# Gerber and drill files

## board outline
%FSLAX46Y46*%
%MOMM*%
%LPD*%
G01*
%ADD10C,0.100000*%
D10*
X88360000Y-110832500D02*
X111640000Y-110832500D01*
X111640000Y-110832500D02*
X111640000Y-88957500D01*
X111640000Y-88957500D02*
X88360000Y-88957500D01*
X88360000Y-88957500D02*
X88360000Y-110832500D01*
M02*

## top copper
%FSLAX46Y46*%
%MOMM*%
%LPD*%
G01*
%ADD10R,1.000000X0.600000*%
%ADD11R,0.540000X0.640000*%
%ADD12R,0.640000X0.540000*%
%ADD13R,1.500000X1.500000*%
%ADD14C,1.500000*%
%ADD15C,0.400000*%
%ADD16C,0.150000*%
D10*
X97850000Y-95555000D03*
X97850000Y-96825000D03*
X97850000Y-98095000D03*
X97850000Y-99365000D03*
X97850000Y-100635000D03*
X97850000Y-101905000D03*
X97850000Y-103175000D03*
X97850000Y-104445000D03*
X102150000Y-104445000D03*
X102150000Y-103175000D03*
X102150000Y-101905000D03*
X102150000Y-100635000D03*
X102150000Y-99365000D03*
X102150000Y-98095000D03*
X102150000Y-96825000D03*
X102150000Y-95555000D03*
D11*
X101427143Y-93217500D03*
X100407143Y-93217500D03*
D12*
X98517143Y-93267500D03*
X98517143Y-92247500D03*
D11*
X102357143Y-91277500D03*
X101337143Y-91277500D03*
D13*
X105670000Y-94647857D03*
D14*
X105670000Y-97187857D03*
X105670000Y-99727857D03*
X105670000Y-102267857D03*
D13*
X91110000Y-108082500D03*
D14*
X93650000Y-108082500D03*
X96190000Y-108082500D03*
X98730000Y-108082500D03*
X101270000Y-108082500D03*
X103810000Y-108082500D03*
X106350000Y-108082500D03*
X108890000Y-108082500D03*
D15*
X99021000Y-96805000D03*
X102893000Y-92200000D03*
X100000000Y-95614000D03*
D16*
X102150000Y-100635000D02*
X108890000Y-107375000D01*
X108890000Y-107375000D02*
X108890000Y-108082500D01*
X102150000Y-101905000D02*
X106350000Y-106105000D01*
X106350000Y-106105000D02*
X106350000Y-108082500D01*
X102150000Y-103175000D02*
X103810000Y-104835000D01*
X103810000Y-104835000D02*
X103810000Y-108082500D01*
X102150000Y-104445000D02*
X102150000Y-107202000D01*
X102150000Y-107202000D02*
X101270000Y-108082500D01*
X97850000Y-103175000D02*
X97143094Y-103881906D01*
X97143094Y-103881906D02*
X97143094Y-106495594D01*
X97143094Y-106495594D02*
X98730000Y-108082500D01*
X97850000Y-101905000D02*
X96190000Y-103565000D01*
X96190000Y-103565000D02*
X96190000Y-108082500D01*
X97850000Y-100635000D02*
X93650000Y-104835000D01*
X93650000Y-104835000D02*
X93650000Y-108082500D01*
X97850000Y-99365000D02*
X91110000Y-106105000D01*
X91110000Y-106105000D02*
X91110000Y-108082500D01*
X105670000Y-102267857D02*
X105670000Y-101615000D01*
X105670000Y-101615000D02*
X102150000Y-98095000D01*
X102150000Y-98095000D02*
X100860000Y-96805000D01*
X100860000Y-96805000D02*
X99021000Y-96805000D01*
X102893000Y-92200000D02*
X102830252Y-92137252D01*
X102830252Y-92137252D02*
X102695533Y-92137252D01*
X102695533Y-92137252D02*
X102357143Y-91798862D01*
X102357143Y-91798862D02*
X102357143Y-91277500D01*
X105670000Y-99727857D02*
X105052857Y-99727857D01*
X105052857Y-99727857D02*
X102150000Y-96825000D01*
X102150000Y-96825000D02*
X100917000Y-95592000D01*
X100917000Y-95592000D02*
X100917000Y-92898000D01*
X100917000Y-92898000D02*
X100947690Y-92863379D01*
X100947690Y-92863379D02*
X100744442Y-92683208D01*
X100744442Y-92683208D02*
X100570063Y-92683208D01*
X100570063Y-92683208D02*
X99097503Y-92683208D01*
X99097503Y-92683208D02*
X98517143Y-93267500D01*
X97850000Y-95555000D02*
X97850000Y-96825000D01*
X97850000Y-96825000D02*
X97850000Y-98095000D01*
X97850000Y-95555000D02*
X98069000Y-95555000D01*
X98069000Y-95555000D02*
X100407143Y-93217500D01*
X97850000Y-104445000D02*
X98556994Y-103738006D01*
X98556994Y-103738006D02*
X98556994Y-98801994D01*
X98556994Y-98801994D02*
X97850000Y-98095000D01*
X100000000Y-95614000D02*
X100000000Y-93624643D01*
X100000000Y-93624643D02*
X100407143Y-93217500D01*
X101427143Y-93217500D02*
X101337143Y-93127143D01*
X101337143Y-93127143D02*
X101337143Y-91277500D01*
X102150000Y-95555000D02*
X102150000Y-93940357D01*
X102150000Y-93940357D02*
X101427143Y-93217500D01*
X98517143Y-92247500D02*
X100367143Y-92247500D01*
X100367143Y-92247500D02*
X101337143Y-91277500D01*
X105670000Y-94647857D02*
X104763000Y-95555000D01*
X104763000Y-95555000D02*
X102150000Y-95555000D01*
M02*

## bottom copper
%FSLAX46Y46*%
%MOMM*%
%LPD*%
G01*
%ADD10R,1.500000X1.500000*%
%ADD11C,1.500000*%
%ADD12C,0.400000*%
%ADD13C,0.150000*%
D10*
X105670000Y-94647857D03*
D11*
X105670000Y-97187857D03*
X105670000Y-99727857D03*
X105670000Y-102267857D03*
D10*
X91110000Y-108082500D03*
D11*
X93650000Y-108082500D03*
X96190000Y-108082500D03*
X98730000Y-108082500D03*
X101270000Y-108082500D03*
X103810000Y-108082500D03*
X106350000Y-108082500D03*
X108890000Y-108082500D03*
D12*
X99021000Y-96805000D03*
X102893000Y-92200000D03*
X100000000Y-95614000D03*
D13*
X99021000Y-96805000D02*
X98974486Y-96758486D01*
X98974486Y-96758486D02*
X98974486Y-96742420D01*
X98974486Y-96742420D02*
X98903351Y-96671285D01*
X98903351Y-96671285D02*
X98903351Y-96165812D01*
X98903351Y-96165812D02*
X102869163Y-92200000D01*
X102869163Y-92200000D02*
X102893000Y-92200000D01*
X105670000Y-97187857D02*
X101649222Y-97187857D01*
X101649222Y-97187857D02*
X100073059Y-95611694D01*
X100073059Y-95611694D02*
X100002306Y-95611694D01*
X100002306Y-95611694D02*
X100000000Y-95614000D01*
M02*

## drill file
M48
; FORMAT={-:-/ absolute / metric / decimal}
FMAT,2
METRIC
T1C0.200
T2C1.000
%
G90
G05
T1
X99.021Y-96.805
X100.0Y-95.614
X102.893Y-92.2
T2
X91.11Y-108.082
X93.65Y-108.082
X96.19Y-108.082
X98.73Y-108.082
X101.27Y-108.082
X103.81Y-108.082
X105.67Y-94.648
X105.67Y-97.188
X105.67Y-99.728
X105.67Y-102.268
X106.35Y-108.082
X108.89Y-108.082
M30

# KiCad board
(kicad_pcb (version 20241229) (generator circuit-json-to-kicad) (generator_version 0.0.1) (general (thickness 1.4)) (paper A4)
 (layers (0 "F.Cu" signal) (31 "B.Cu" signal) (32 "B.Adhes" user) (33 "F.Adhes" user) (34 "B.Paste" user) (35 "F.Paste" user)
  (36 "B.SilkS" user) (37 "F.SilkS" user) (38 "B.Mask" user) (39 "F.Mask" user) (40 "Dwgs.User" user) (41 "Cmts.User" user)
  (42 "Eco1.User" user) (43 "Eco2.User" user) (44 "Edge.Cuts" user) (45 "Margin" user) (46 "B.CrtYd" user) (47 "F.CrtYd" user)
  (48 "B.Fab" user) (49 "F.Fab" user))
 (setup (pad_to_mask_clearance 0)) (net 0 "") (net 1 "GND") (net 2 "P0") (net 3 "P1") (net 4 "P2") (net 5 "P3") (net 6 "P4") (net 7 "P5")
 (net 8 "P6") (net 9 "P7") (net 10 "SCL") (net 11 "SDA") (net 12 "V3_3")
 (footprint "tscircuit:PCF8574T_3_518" (layer F.Cu) (at 100 100 0)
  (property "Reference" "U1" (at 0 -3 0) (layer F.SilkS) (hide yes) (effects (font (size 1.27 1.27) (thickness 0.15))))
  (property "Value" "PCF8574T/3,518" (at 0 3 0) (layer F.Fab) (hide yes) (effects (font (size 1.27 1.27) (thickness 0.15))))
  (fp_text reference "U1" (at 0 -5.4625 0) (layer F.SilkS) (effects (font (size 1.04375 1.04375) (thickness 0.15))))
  (pad "1" smd rect (at -2.15 -4.445 0) (size 1 0.6) (layers F.Cu F.Paste F.Mask) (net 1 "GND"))
  (pad "2" smd rect (at -2.15 -3.1750000000000003 0) (size 1 0.6) (layers F.Cu F.Paste F.Mask) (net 1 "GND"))
  (pad "3" smd rect (at -2.15 -1.9050000000000002 0) (size 1 0.6) (layers F.Cu F.Paste F.Mask) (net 1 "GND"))
  (pad "4" smd rect (at -2.15 -0.6350000000000002 0) (size 1 0.6) (layers F.Cu F.Paste F.Mask) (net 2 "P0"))
  (pad "5" smd rect (at -2.15 0.6349999999999998 0) (size 1 0.6) (layers F.Cu F.Paste F.Mask) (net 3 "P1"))
  (pad "6" smd rect (at -2.15 1.9049999999999994 0) (size 1 0.6) (layers F.Cu F.Paste F.Mask) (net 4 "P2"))
  (pad "7" smd rect (at -2.15 3.175 0) (size 1 0.6) (layers F.Cu F.Paste F.Mask) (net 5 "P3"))
  (pad "8" smd rect (at -2.15 4.445 0) (size 1 0.6) (layers F.Cu F.Paste F.Mask) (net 1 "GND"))
  (pad "9" smd rect (at 2.15 4.445 0) (size 1 0.6) (layers F.Cu F.Paste F.Mask) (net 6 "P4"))
  (pad "10" smd rect (at 2.15 3.1750000000000003 0) (size 1 0.6) (layers F.Cu F.Paste F.Mask) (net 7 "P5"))
  (pad "11" smd rect (at 2.15 1.9050000000000002 0) (size 1 0.6) (layers F.Cu F.Paste F.Mask) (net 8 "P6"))
  (pad "12" smd rect (at 2.15 0.6350000000000002 0) (size 1 0.6) (layers F.Cu F.Paste F.Mask) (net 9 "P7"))
  (pad "13" smd rect (at 2.15 -0.6349999999999998 0) (size 1 0.6) (layers F.Cu F.Paste F.Mask))
  (pad "14" smd rect (at 2.15 -1.9049999999999994 0) (size 1 0.6) (layers F.Cu F.Paste F.Mask) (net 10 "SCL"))
  (pad "15" smd rect (at 2.15 -3.175 0) (size 1 0.6) (layers F.Cu F.Paste F.Mask) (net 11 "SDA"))
  (pad "16" smd rect (at 2.15 -4.445 0) (size 1 0.6) (layers F.Cu F.Paste F.Mask) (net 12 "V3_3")))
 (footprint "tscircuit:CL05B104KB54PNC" (layer F.Cu) (at 100.91714285714286 93.2175 180)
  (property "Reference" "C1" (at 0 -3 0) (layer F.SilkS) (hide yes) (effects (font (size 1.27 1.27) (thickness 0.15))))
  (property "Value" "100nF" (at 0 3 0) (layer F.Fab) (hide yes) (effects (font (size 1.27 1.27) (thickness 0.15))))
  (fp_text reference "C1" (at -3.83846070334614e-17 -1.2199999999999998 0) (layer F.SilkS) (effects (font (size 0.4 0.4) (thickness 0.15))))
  (pad "1" smd rect (at -0.5099999999999999 0 0) (size 0.54 0.64) (layers F.Cu F.Paste F.Mask) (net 12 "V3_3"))
  (pad "2" smd rect (at 0.51 0 0) (size 0.54 0.64) (layers F.Cu F.Paste F.Mask) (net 1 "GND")))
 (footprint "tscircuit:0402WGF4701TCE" (layer F.Cu) (at 98.51714285714286 92.7575 90)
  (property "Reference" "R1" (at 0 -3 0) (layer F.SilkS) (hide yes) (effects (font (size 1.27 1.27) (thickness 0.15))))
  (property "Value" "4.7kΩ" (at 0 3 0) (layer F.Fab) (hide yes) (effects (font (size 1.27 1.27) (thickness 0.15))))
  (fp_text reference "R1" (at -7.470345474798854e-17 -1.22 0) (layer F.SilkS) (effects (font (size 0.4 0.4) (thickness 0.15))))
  (pad "1" smd rect (at -0.5099999999999998 0 0) (size 0.64 0.54) (layers F.Cu F.Paste F.Mask) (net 11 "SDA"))
  (pad "2" smd rect (at 0.5099999999999998 0 0) (size 0.64 0.54) (layers F.Cu F.Paste F.Mask) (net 12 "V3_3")))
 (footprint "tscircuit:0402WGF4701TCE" (layer F.Cu) (at 101.84714285714286 91.2775 180)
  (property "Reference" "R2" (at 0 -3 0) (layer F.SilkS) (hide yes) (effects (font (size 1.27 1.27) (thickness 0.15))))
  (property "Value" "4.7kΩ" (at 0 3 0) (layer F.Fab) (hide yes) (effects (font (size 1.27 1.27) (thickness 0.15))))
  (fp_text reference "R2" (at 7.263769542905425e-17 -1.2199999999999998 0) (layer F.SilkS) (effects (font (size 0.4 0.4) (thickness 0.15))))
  (pad "1" smd rect (at -0.51 0 0) (size 0.54 0.64) (layers F.Cu F.Paste F.Mask) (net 10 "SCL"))
  (pad "2" smd rect (at 0.51 0 0) (size 0.54 0.64) (layers F.Cu F.Paste F.Mask) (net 12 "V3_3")))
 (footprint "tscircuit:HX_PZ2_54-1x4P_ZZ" (layer F.Cu) (at 105.67 98.45785714285714 -90.00000000000001)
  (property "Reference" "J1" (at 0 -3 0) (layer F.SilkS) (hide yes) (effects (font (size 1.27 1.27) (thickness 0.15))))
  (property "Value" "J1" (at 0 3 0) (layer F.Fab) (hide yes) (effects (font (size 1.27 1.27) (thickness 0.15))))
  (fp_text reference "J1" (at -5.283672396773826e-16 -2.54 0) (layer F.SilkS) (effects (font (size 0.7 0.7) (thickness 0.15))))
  (pad "1" thru_hole rect (at -3.81 5.705062545910424e-16 0) (size 1.5 1.5) (drill 1) (layers *.Cu *.Mask) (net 12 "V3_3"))
  (pad "2" thru_hole circle (at -1.27 4.862282247637226e-16 0) (size 1.5 1.5) (drill 1) (layers *.Cu *.Mask) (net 1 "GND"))
  (pad "3" thru_hole circle (at 1.27 -4.862282247637226e-16 0) (size 1.5 1.5) (drill 1) (layers *.Cu *.Mask) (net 11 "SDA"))
  (pad "4" thru_hole circle (at 3.81 -5.705062545910424e-16 0) (size 1.5 1.5) (drill 1) (layers *.Cu *.Mask) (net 10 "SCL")))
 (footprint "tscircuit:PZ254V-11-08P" (layer F.Cu) (at 100 108.0825 0)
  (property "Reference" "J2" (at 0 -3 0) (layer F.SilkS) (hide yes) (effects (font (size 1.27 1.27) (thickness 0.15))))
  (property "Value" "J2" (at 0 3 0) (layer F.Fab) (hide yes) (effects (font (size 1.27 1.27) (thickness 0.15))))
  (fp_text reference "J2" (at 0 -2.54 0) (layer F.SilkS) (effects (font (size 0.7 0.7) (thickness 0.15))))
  (pad "1" thru_hole rect (at -8.89 0 0) (size 1.5 1.5) (drill 1) (layers *.Cu *.Mask) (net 2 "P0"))
  (pad "2" thru_hole circle (at -6.3500000000000005 0 0) (size 1.5 1.5) (drill 1) (layers *.Cu *.Mask) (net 3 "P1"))
  (pad "3" thru_hole circle (at -3.8100000000000005 0 0) (size 1.5 1.5) (drill 1) (layers *.Cu *.Mask) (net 4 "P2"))
  (pad "4" thru_hole circle (at -1.2700000000000005 0 0) (size 1.5 1.5) (drill 1) (layers *.Cu *.Mask) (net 5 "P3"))
  (pad "5" thru_hole circle (at 1.2699999999999996 0 0) (size 1.5 1.5) (drill 1) (layers *.Cu *.Mask) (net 6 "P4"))
  (pad "6" thru_hole circle (at 3.8099999999999987 0 0) (size 1.5 1.5) (drill 1) (layers *.Cu *.Mask) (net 7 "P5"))
  (pad "7" thru_hole circle (at 6.35 0 0) (size 1.5 1.5) (drill 1) (layers *.Cu *.Mask) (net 8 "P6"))
  (pad "8" thru_hole circle (at 8.89 0 0) (size 1.5 1.5) (drill 1) (layers *.Cu *.Mask) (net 9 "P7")))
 (segment (start 102.15 100.635) (end 108.89 107.375) (width 0.15) (layer F.Cu) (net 9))
 (segment (start 108.89 107.375) (end 108.89 108.0825) (width 0.15) (layer F.Cu) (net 9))
 (segment (start 102.15 101.905) (end 106.35 106.105) (width 0.15) (layer F.Cu) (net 8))
 (segment (start 106.35 106.105) (end 106.35 108.0825) (width 0.15) (layer F.Cu) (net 8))
 (segment (start 102.15 103.175) (end 103.81 104.835) (width 0.15) (layer F.Cu) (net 7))
 (segment (start 103.81 104.835) (end 103.81 108.0825) (width 0.15) (layer F.Cu) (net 7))
 (segment (start 102.15 104.445) (end 102.15 107.202) (width 0.15) (layer F.Cu) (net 6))
 (segment (start 102.15 107.202) (end 101.27 108.0825) (width 0.15) (layer F.Cu) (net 6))
 (segment (start 97.85 103.175) (end 97.14309387785406 103.88190612214595) (width 0.15) (layer F.Cu) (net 5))
 (segment (start 97.14309387785406 103.88190612214595) (end 97.14309387785406 106.49559387785405) (width 0.15) (layer F.Cu) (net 5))
 (segment (start 97.14309387785406 106.49559387785405) (end 98.73 108.0825) (width 0.15) (layer F.Cu) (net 5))
 (segment (start 97.85 101.905) (end 96.19 103.565) (width 0.15) (layer F.Cu) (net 4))
 (segment (start 96.19 103.565) (end 96.19 108.0825) (width 0.15) (layer F.Cu) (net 4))
 (segment (start 97.85 100.635) (end 93.65 104.83500000000001) (width 0.15) (layer F.Cu) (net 3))
 (segment (start 93.65 104.83500000000001) (end 93.65 108.0825) (width 0.15) (layer F.Cu) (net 3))
 (segment (start 97.85 99.365) (end 91.11 106.105) (width 0.15) (layer F.Cu) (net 2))
 (segment (start 91.11 106.105) (end 91.11 108.0825) (width 0.15) (layer F.Cu) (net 2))
 (segment (start 105.67 102.26785714285714) (end 105.67 101.615) (width 0.15) (layer F.Cu) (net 10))
 (segment (start 105.67 101.615) (end 102.15 98.095) (width 0.15) (layer F.Cu) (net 10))
 (segment (start 102.15 98.095) (end 100.86 96.805) (width 0.15) (layer F.Cu) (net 10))
 (segment (start 100.86 96.805) (end 99.021 96.805) (width 0.15) (layer F.Cu) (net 10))
 (segment (start 99.021 96.805) (end 98.97448570689265 96.75848570689264) (width 0.15) (layer B.Cu) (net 10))
 (segment (start 98.97448570689265 96.75848570689264) (end 98.97448570689265 96.7424195752621) (width 0.15) (layer B.Cu) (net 10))
 (segment (start 98.97448570689265 96.7424195752621) (end 98.90335073935582 96.67128460772527) (width 0.15) (layer B.Cu) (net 10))
 (segment (start 98.90335073935582 96.67128460772527) (end 98.90335073935582 96.1658122704005) (width 0.15) (layer B.Cu) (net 10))
 (segment (start 98.90335073935582 96.1658122704005) (end 102.86916300975629 92.2) (width 0.15) (layer B.Cu) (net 10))
 (segment (start 102.86916300975629 92.2) (end 102.893 92.2) (width 0.15) (layer B.Cu) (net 10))
 (segment (start 102.893 92.2) (end 102.83025181571226 92.13725181571226) (width 0.15) (layer F.Cu) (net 10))
 (segment (start 102.83025181571226 92.13725181571226) (end 102.69553276752963 92.13725181571226) (width 0.15) (layer F.Cu) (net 10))
 (segment (start 102.69553276752963 92.13725181571226) (end 102.35714285714286 91.7988619053255) (width 0.15) (layer F.Cu) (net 10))
 (segment (start 102.35714285714286 91.7988619053255) (end 102.35714285714286 91.2775) (width 0.15) (layer F.Cu) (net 10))
 (segment (start 105.67 99.72785714285715) (end 105.05285714285714 99.72785714285715) (width 0.15) (layer F.Cu) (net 11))
 (segment (start 105.05285714285714 99.72785714285715) (end 102.15 96.825) (width 0.15) (layer F.Cu) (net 11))
 (segment (start 102.15 96.825) (end 100.917 95.592) (width 0.15) (layer F.Cu) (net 11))
 (segment (start 100.917 95.592) (end 100.917 92.898) (width 0.15) (layer F.Cu) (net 11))
 (segment (start 100.917 92.898) (end 100.9476902638268 92.8633786928267) (width 0.15) (layer F.Cu) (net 11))
 (segment (start 100.9476902638268 92.8633786928267) (end 100.7444423942015 92.68320840896624) (width 0.15) (layer F.Cu) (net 11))
 (segment (start 100.7444423942015 92.68320840896624) (end 100.57006282266266 92.68320840896624) (width 0.15) (layer F.Cu) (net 11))
 (segment (start 100.57006282266266 92.68320840896624) (end 99.09750340483012 92.68320840896624) (width 0.15) (layer F.Cu) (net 11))
 (segment (start 99.09750340483012 92.68320840896624) (end 98.51714285714286 93.2675) (width 0.15) (layer F.Cu) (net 11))
 (segment (start 97.85 95.555) (end 97.85 96.825) (width 0.15) (layer F.Cu) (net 1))
 (segment (start 97.85 96.825) (end 97.85 98.095) (width 0.15) (layer F.Cu) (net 1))
 (segment (start 97.85 95.555) (end 98.069 95.555) (width 0.15) (layer F.Cu) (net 1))
 (segment (start 98.069 95.555) (end 100.40714285714286 93.2175) (width 0.15) (layer F.Cu) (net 1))
 (segment (start 97.85 104.445) (end 98.55699418028716 103.73800581971284) (width 0.15) (layer F.Cu) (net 1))
 (segment (start 98.55699418028716 103.73800581971284) (end 98.55699418028716 98.80199418028717) (width 0.15) (layer F.Cu) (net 1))
 (segment (start 98.55699418028716 98.80199418028717) (end 97.85 98.095) (width 0.15) (layer F.Cu) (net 1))
 (segment (start 105.67 97.18785714285714) (end 101.64922166590743 97.18785714285714) (width 0.15) (layer B.Cu) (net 1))
 (segment (start 101.64922166590743 97.18785714285714) (end 100.07305874681478 95.6116942237645) (width 0.15) (layer B.Cu) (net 1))
 (segment (start 100.07305874681478 95.6116942237645) (end 100.0023057762355 95.6116942237645) (width 0.15) (layer B.Cu) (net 1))
 (segment (start 100.0023057762355 95.6116942237645) (end 100 95.614) (width 0.15) (layer B.Cu) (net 1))
 (segment (start 100 95.614) (end 100 93.62464285714286) (width 0.15) (layer F.Cu) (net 1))
 (segment (start 100 93.62464285714286) (end 100.40714285714286 93.2175) (width 0.15) (layer F.Cu) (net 1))
 (segment (start 101.42714285714285 93.2175) (end 101.33714285714285 93.12714285714286) (width 0.15) (layer F.Cu) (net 12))
 (segment (start 101.33714285714285 93.12714285714286) (end 101.33714285714285 91.2775) (width 0.15) (layer F.Cu) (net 12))
 (segment (start 102.15 95.555) (end 102.15 93.94035714285714) (width 0.15) (layer F.Cu) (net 12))
 (segment (start 102.15 93.94035714285714) (end 101.42714285714285 93.2175) (width 0.15) (layer F.Cu) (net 12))
 (segment (start 98.51714285714286 92.2475) (end 100.36714285714285 92.2475) (width 0.15) (layer F.Cu) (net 12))
 (segment (start 100.36714285714285 92.2475) (end 101.33714285714285 91.2775) (width 0.15) (layer F.Cu) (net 12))
 (segment (start 105.67 94.64785714285715) (end 104.763 95.555) (width 0.15) (layer F.Cu) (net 12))
 (segment (start 104.763 95.555) (end 102.15 95.555) (width 0.15) (layer F.Cu) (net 12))
 (gr_line (start 88.36 110.8325) (end 111.64 110.8325) (width 0.1) (layer Edge.Cuts))
 (gr_line (start 111.64 110.8325) (end 111.64 88.9575) (width 0.1) (layer Edge.Cuts))
 (gr_line (start 111.64 88.9575) (end 88.36 88.9575) (width 0.1) (layer Edge.Cuts))
 (gr_line (start 88.36 88.9575) (end 88.36 110.8325) (width 0.1) (layer Edge.Cuts))
 (via (at 99.021 96.805) (size 0.4) (drill 0.2) (layers F.Cu B.Cu) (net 10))
 (via (at 102.893 92.2) (size 0.4) (drill 0.2) (layers F.Cu B.Cu) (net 10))
 (via (at 100 95.614) (size 0.4) (drill 0.2) (layers F.Cu B.Cu) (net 1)))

